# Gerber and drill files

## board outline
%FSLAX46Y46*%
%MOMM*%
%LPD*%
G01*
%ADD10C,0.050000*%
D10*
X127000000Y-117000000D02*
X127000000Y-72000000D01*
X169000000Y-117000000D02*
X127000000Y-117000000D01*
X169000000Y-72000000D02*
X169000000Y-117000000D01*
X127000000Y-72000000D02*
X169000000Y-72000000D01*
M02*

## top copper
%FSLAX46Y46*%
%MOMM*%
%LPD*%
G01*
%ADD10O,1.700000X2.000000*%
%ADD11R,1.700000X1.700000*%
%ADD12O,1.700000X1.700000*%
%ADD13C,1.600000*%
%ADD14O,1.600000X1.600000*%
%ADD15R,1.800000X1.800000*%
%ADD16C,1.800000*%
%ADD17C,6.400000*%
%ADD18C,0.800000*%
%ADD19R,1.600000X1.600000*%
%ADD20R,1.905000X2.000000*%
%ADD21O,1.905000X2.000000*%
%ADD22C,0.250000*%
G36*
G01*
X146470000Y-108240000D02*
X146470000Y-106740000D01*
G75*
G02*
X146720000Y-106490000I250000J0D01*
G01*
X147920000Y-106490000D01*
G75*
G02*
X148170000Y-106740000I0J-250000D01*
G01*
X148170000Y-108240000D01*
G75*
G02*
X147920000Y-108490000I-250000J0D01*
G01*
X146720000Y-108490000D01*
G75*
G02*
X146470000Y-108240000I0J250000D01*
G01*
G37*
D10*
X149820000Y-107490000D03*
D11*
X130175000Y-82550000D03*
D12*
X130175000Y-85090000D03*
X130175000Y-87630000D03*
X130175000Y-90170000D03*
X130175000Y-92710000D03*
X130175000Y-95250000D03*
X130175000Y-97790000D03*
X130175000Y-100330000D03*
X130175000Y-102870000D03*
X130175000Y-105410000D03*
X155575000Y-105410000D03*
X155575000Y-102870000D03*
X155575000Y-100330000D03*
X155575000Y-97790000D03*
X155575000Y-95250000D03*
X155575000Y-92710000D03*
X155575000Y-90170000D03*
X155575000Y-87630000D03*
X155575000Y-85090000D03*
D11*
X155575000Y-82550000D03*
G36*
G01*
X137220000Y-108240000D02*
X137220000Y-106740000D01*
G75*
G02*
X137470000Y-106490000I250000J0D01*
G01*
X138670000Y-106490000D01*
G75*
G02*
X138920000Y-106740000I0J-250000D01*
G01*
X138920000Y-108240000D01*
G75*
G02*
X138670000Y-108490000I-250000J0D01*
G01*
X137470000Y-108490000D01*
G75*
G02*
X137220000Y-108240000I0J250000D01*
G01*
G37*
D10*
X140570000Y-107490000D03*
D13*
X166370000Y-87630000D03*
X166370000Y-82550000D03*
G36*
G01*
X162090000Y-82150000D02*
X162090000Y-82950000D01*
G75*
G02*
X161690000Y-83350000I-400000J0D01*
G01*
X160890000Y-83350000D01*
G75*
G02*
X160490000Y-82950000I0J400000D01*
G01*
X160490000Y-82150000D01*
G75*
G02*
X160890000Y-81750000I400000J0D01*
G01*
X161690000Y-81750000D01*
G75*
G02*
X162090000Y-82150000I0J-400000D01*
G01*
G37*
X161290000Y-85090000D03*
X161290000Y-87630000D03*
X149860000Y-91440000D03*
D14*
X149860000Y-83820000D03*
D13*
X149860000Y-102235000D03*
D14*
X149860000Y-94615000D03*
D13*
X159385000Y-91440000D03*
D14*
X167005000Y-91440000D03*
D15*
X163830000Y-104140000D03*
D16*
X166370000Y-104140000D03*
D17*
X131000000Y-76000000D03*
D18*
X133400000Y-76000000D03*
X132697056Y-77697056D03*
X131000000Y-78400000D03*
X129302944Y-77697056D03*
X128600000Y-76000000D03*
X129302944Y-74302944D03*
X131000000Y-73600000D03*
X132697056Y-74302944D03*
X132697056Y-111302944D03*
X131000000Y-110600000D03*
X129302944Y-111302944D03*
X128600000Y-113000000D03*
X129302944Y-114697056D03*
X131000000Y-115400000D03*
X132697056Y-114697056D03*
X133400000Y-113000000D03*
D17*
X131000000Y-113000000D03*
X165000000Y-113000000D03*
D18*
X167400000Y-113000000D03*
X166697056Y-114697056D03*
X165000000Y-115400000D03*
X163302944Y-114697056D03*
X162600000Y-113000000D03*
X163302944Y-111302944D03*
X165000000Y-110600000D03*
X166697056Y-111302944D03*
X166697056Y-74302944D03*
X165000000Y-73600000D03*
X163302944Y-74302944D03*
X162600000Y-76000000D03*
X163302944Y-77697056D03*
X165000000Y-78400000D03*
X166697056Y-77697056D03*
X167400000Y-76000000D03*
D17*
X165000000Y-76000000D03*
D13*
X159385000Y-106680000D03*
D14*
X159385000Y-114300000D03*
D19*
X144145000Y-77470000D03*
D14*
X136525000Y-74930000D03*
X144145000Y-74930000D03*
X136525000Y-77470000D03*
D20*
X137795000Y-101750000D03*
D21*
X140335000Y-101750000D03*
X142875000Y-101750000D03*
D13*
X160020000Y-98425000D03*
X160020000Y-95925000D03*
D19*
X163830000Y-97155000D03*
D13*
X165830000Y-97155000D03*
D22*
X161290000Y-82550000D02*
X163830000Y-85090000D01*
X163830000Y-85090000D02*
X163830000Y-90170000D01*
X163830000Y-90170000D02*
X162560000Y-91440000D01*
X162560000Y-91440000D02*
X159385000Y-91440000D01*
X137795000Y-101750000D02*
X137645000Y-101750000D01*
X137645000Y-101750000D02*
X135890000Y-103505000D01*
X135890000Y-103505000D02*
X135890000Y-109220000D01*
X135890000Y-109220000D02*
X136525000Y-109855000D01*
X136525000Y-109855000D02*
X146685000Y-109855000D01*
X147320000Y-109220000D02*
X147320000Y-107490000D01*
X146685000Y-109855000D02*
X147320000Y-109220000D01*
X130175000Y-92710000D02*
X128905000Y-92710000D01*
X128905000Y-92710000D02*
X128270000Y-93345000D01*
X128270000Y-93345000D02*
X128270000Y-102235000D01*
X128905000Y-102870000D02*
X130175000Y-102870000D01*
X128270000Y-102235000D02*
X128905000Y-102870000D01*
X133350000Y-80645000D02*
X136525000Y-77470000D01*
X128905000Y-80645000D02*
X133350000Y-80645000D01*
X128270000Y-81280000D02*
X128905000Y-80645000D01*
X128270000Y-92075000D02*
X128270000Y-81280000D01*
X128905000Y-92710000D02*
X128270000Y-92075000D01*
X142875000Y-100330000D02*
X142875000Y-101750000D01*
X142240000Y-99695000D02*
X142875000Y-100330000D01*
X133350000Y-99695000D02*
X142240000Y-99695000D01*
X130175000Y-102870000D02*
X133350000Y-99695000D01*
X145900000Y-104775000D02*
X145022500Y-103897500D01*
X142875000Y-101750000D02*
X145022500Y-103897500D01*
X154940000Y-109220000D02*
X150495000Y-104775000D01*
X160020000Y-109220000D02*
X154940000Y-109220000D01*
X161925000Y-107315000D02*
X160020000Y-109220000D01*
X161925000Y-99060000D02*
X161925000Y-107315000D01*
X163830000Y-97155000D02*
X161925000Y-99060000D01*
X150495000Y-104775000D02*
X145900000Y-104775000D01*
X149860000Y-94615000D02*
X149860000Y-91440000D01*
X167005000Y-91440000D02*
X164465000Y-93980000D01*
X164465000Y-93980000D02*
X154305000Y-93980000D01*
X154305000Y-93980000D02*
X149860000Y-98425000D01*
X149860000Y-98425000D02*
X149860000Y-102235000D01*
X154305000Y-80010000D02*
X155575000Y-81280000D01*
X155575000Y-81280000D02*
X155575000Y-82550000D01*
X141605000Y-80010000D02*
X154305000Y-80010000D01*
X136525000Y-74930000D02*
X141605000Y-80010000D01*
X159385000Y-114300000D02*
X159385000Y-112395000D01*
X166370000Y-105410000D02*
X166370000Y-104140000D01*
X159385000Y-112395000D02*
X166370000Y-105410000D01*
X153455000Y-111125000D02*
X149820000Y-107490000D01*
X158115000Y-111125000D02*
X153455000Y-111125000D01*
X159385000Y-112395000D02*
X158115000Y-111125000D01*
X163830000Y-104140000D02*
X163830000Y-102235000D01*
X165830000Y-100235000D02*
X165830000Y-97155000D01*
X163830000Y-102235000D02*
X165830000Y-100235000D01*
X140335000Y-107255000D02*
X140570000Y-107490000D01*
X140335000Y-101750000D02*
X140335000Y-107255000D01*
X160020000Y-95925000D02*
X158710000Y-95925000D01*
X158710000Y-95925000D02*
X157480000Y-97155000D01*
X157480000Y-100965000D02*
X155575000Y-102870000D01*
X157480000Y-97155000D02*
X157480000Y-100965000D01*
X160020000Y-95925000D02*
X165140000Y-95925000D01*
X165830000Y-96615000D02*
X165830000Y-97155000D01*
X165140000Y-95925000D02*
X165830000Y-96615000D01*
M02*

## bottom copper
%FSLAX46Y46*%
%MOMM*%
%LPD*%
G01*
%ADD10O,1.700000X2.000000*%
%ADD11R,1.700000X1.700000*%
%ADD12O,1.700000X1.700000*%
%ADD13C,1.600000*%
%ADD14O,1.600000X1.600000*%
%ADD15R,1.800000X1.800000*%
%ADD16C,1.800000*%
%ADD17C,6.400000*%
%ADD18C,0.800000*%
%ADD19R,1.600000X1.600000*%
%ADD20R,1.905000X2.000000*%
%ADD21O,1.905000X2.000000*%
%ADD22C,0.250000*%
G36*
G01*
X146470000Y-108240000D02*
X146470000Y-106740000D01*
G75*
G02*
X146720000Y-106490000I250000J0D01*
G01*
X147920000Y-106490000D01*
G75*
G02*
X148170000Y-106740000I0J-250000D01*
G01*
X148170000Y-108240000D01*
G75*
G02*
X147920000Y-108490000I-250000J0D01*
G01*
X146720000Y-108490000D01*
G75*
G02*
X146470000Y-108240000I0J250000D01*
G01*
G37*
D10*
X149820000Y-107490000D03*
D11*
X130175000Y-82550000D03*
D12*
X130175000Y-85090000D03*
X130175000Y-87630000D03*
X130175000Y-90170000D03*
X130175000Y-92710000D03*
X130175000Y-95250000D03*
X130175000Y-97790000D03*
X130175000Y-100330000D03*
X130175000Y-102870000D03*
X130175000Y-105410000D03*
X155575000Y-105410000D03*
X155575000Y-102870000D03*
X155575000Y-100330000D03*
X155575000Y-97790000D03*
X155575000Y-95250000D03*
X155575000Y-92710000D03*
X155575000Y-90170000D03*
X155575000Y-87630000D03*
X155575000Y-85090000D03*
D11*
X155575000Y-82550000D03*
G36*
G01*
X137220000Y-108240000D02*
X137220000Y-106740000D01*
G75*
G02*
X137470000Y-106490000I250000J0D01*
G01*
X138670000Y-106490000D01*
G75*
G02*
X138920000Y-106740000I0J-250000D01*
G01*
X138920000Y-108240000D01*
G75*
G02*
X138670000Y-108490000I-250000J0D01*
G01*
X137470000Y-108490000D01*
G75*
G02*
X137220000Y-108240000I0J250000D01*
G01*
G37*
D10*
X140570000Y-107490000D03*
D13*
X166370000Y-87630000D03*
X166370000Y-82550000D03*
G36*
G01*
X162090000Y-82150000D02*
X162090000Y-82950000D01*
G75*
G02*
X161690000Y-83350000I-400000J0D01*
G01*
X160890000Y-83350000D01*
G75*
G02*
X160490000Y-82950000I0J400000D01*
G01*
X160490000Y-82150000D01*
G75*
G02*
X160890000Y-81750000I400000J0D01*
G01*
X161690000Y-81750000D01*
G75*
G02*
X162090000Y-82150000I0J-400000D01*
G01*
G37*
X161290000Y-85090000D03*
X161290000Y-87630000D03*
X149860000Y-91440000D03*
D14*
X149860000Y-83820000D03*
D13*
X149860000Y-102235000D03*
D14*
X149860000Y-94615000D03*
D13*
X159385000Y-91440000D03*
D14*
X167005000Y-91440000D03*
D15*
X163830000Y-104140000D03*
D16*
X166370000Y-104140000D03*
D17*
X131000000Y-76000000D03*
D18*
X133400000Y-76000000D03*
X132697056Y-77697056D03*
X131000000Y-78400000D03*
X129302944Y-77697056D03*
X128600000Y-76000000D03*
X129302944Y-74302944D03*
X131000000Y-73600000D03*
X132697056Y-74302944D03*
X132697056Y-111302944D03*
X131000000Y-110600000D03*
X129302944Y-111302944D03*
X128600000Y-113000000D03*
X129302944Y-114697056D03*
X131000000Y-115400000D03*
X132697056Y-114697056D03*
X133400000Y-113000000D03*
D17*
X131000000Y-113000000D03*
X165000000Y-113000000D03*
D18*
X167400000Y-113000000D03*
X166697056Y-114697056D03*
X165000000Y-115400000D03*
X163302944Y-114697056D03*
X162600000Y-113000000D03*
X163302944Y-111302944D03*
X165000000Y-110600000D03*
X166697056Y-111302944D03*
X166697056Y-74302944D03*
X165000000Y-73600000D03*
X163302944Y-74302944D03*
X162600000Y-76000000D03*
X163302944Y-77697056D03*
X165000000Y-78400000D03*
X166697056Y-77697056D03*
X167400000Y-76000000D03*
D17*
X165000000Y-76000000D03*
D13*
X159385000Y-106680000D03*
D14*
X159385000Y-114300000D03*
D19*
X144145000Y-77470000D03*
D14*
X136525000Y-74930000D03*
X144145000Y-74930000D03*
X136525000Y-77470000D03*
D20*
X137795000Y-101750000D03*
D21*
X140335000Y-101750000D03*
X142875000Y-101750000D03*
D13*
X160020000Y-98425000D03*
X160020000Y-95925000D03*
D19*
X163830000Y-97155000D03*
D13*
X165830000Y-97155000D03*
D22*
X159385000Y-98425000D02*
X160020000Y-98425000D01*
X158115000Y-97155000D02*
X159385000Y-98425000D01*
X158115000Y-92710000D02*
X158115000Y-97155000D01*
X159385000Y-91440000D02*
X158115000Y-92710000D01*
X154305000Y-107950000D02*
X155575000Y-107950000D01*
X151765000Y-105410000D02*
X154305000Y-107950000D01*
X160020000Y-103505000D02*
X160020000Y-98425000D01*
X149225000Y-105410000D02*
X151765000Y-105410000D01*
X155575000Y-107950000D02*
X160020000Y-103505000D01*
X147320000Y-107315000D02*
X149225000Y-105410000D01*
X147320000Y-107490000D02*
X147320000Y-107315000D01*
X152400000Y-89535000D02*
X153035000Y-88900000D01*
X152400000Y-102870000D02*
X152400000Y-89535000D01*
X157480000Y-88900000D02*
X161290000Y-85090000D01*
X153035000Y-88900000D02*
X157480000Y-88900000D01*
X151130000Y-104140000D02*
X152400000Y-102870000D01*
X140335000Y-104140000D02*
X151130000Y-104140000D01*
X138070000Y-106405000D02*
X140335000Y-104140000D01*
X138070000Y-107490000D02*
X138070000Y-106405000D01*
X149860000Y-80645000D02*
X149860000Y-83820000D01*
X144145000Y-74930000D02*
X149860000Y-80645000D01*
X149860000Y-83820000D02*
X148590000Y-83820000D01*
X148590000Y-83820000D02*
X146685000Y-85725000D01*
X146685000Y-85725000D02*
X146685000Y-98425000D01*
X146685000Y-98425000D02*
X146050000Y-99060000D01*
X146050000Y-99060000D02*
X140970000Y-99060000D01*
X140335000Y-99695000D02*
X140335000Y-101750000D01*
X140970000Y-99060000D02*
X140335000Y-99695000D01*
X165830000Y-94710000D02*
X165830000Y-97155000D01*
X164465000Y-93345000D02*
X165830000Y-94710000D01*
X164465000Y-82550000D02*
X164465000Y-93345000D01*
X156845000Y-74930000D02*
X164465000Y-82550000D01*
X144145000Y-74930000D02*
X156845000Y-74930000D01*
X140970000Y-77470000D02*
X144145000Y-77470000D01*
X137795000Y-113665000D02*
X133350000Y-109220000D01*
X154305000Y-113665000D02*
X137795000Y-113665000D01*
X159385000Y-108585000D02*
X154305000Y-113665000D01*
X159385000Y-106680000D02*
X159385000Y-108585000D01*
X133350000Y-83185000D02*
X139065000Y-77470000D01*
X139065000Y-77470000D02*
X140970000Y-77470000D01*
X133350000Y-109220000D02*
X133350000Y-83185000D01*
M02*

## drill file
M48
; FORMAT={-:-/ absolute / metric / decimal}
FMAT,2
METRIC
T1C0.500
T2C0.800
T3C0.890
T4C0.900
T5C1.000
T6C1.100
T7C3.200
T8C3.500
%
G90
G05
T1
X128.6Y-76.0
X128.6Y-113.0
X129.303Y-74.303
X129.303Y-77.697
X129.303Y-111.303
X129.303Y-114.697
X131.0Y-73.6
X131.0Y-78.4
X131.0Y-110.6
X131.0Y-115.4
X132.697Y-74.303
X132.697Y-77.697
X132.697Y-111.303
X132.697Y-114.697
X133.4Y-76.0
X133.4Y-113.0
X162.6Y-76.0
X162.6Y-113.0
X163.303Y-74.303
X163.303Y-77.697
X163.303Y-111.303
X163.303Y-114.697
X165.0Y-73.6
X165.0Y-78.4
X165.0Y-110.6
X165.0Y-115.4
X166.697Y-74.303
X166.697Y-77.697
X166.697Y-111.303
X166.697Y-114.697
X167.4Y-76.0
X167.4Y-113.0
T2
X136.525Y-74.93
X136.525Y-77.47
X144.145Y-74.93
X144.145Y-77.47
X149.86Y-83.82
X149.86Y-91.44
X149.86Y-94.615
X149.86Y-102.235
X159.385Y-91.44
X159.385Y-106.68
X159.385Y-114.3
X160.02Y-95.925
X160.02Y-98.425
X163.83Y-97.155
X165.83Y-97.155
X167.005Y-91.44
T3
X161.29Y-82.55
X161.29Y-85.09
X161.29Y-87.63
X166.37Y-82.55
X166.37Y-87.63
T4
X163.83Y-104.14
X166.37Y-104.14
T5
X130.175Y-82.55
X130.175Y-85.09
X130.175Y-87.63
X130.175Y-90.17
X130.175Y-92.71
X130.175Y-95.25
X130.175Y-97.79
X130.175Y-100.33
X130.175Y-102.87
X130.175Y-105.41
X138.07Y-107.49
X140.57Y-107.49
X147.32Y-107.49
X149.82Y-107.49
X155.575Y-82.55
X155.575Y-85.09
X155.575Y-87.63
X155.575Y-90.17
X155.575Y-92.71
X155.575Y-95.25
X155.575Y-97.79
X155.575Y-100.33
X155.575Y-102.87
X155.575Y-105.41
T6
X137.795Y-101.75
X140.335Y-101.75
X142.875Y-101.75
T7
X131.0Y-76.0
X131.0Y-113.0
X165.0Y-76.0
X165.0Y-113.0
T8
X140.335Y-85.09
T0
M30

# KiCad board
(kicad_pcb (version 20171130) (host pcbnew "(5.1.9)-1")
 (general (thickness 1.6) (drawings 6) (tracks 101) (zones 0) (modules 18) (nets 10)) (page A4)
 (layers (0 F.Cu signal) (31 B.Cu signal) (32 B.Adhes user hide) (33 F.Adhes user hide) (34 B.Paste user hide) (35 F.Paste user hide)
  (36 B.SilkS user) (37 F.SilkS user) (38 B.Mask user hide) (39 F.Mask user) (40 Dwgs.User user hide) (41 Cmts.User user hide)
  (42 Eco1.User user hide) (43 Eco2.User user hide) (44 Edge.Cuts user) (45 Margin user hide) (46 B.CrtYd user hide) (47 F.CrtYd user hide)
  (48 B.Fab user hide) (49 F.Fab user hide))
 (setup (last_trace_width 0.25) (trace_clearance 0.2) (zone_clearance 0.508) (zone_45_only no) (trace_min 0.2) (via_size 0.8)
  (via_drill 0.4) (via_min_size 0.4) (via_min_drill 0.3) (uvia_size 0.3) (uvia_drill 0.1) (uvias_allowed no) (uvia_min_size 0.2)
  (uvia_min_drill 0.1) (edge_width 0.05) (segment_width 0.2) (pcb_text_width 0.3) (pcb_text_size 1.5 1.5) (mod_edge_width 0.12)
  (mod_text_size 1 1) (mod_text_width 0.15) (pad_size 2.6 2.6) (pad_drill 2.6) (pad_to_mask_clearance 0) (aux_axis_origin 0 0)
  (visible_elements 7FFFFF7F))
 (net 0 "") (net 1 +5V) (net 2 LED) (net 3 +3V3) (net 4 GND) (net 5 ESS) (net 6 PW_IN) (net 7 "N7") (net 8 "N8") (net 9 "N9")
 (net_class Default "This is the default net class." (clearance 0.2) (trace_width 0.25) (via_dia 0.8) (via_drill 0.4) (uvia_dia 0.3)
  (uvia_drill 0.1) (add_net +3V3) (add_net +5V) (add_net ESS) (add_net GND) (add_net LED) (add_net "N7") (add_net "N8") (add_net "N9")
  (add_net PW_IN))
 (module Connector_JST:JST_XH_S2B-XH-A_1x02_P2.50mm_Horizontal (layer F.Cu) (at 147.32 107.49)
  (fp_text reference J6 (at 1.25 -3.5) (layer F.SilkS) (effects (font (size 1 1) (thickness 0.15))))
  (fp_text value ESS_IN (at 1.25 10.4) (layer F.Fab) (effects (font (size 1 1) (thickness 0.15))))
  (pad 1 thru_hole roundrect (at 0 0) (size 1.7 2) (drill 1) (layers *.Cu *.Mask) (roundrect_rratio 0.1470588235294118) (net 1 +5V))
  (pad 2 thru_hole oval (at 2.5 0) (size 1.7 2) (drill 1) (layers *.Cu *.Mask) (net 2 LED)))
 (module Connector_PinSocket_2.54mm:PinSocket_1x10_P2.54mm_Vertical (layer F.Cu) (at 130.175 82.55)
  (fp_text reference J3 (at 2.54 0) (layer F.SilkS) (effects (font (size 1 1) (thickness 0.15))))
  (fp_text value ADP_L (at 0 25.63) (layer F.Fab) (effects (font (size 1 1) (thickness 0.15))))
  (pad 1 thru_hole rect (at 0 0) (size 1.7 1.7) (drill 1) (layers *.Cu *.Mask))
  (pad 2 thru_hole oval (at 0 2.54) (size 1.7 1.7) (drill 1) (layers *.Cu *.Mask))
  (pad 3 thru_hole oval (at 0 5.08) (size 1.7 1.7) (drill 1) (layers *.Cu *.Mask))
  (pad 4 thru_hole oval (at 0 7.62) (size 1.7 1.7) (drill 1) (layers *.Cu *.Mask))
  (pad 5 thru_hole oval (at 0 10.16) (size 1.7 1.7) (drill 1) (layers *.Cu *.Mask) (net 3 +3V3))
  (pad 6 thru_hole oval (at 0 12.7) (size 1.7 1.7) (drill 1) (layers *.Cu *.Mask))
  (pad 7 thru_hole oval (at 0 15.24) (size 1.7 1.7) (drill 1) (layers *.Cu *.Mask))
  (pad 8 thru_hole oval (at 0 17.78) (size 1.7 1.7) (drill 1) (layers *.Cu *.Mask))
  (pad 9 thru_hole oval (at 0 20.32) (size 1.7 1.7) (drill 1) (layers *.Cu *.Mask) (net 3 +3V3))
  (pad 10 thru_hole oval (at 0 22.86) (size 1.7 1.7) (drill 1) (layers *.Cu *.Mask)))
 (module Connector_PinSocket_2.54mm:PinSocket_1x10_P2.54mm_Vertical (layer F.Cu) (at 155.575 82.55)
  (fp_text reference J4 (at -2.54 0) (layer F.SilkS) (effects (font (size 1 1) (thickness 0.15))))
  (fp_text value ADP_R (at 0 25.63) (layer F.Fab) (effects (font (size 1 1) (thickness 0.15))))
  (pad 10 thru_hole oval (at 0 22.86) (size 1.7 1.7) (drill 1) (layers *.Cu *.Mask))
  (pad 9 thru_hole oval (at 0 20.32) (size 1.7 1.7) (drill 1) (layers *.Cu *.Mask) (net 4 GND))
  (pad 8 thru_hole oval (at 0 17.78) (size 1.7 1.7) (drill 1) (layers *.Cu *.Mask))
  (pad 7 thru_hole oval (at 0 15.24) (size 1.7 1.7) (drill 1) (layers *.Cu *.Mask))
  (pad 6 thru_hole oval (at 0 12.7) (size 1.7 1.7) (drill 1) (layers *.Cu *.Mask))
  (pad 5 thru_hole oval (at 0 10.16) (size 1.7 1.7) (drill 1) (layers *.Cu *.Mask))
  (pad 4 thru_hole oval (at 0 7.62) (size 1.7 1.7) (drill 1) (layers *.Cu *.Mask))
  (pad 3 thru_hole oval (at 0 5.08) (size 1.7 1.7) (drill 1) (layers *.Cu *.Mask))
  (pad 2 thru_hole oval (at 0 2.54) (size 1.7 1.7) (drill 1) (layers *.Cu *.Mask))
  (pad 1 thru_hole rect (at 0 0) (size 1.7 1.7) (drill 1) (layers *.Cu *.Mask) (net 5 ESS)))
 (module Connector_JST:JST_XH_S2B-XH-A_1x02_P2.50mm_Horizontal (layer F.Cu) (at 138.07 107.49)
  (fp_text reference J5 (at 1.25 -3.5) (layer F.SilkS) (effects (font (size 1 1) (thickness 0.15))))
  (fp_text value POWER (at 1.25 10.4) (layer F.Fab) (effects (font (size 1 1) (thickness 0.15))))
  (pad 1 thru_hole roundrect (at 0 0) (size 1.7 2) (drill 1) (layers *.Cu *.Mask) (roundrect_rratio 0.1470588235294118) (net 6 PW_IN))
  (pad 2 thru_hole oval (at 2.5 0) (size 1.7 2) (drill 1) (layers *.Cu *.Mask) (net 4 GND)))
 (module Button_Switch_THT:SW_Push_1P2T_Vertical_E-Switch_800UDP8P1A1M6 (layer F.Cu) (at 161.29 82.55)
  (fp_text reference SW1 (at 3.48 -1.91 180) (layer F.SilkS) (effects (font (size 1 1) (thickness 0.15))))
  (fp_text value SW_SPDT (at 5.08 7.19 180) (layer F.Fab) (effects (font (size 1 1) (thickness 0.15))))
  (pad "" thru_hole circle (at 5.08 5.08 180) (size 1.6 1.6) (drill 0.89) (layers *.Cu *.Mask))
  (pad "" thru_hole circle (at 5.08 0 180) (size 1.6 1.6) (drill 0.89) (layers *.Cu *.Mask))
  (pad 1 thru_hole roundrect (at 0 0 180) (size 1.6 1.6) (drill 0.89) (layers *.Cu *.Mask) (roundrect_rratio 0.25) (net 1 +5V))
  (pad 2 thru_hole circle (at 0 2.54 180) (size 1.6 1.6) (drill 0.89) (layers *.Cu *.Mask) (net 6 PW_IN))
  (pad 3 thru_hole circle (at 0 5.08 180) (size 1.6 1.6) (drill 0.89) (layers *.Cu *.Mask)))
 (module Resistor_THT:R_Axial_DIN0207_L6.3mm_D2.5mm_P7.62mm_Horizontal (layer F.Cu) (at 149.86 91.44 90)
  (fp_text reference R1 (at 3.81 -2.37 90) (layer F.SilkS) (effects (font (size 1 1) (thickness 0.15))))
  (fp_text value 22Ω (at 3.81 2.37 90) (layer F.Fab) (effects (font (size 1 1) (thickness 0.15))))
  (pad 1 thru_hole circle (at 0 0 90) (size 1.6 1.6) (drill 0.8) (layers *.Cu *.Mask) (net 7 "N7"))
  (pad 2 thru_hole oval (at 7.62 0 90) (size 1.6 1.6) (drill 0.8) (layers *.Cu *.Mask) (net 4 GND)))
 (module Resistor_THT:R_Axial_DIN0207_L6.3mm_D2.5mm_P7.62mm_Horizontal (layer F.Cu) (at 149.86 102.235 90)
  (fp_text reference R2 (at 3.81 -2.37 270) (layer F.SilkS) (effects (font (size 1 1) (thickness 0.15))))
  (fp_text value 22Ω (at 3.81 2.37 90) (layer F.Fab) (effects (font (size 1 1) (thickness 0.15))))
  (pad 1 thru_hole circle (at 0 0 90) (size 1.6 1.6) (drill 0.8) (layers *.Cu *.Mask) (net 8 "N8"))
  (pad 2 thru_hole oval (at 7.62 0 90) (size 1.6 1.6) (drill 0.8) (layers *.Cu *.Mask) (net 7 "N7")))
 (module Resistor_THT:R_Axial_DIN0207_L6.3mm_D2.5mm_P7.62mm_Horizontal (layer F.Cu) (at 159.385 91.44)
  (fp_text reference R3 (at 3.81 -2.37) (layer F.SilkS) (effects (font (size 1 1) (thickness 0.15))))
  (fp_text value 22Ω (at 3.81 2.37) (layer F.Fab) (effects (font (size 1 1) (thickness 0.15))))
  (pad 1 thru_hole circle (at 0 0) (size 1.6 1.6) (drill 0.8) (layers *.Cu *.Mask) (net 1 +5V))
  (pad 2 thru_hole oval (at 7.62 0) (size 1.6 1.6) (drill 0.8) (layers *.Cu *.Mask) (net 8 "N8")))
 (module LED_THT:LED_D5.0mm (layer F.Cu) (at 163.83 104.14)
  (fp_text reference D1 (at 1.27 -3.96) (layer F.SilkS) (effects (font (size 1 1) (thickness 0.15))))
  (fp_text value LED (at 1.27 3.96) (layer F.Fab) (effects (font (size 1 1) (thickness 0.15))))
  (pad 1 thru_hole rect (at 0 0) (size 1.8 1.8) (drill 0.9) (layers *.Cu *.Mask) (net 4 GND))
  (pad 2 thru_hole circle (at 2.54 0) (size 1.8 1.8) (drill 0.9) (layers *.Cu *.Mask) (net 2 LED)))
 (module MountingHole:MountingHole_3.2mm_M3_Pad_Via (layer F.Cu) (at 131 76)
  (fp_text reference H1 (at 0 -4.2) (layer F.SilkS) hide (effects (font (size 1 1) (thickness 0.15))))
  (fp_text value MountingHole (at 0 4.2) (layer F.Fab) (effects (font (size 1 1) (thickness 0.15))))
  (pad 1 thru_hole circle (at 0 0) (size 6.4 6.4) (drill 3.2) (layers *.Cu *.Mask))
  (pad 1 thru_hole circle (at 2.4 0) (size 0.8 0.8) (drill 0.5) (layers *.Cu *.Mask))
  (pad 1 thru_hole circle (at 1.697056 1.697056) (size 0.8 0.8) (drill 0.5) (layers *.Cu *.Mask))
  (pad 1 thru_hole circle (at 0 2.4) (size 0.8 0.8) (drill 0.5) (layers *.Cu *.Mask))
  (pad 1 thru_hole circle (at -1.697056 1.697056) (size 0.8 0.8) (drill 0.5) (layers *.Cu *.Mask))
  (pad 1 thru_hole circle (at -2.4 0) (size 0.8 0.8) (drill 0.5) (layers *.Cu *.Mask))
  (pad 1 thru_hole circle (at -1.697056 -1.697056) (size 0.8 0.8) (drill 0.5) (layers *.Cu *.Mask))
  (pad 1 thru_hole circle (at 0 -2.4) (size 0.8 0.8) (drill 0.5) (layers *.Cu *.Mask))
  (pad 1 thru_hole circle (at 1.697056 -1.697056) (size 0.8 0.8) (drill 0.5) (layers *.Cu *.Mask)))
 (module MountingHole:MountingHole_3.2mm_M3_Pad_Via (layer F.Cu) (at 131 113)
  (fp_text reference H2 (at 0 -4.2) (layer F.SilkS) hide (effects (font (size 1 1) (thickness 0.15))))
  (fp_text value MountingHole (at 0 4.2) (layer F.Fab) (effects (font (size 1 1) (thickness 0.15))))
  (pad 1 thru_hole circle (at 1.697056 -1.697056) (size 0.8 0.8) (drill 0.5) (layers *.Cu *.Mask))
  (pad 1 thru_hole circle (at 0 -2.4) (size 0.8 0.8) (drill 0.5) (layers *.Cu *.Mask))
  (pad 1 thru_hole circle (at -1.697056 -1.697056) (size 0.8 0.8) (drill 0.5) (layers *.Cu *.Mask))
  (pad 1 thru_hole circle (at -2.4 0) (size 0.8 0.8) (drill 0.5) (layers *.Cu *.Mask))
  (pad 1 thru_hole circle (at -1.697056 1.697056) (size 0.8 0.8) (drill 0.5) (layers *.Cu *.Mask))
  (pad 1 thru_hole circle (at 0 2.4) (size 0.8 0.8) (drill 0.5) (layers *.Cu *.Mask))
  (pad 1 thru_hole circle (at 1.697056 1.697056) (size 0.8 0.8) (drill 0.5) (layers *.Cu *.Mask))
  (pad 1 thru_hole circle (at 2.4 0) (size 0.8 0.8) (drill 0.5) (layers *.Cu *.Mask))
  (pad 1 thru_hole circle (at 0 0) (size 6.4 6.4) (drill 3.2) (layers *.Cu *.Mask)))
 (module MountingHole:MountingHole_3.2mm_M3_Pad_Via (layer F.Cu) (at 165 113)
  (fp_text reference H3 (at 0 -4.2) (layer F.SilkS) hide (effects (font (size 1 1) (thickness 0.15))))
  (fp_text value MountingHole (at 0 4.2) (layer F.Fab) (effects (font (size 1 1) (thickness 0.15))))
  (pad 1 thru_hole circle (at 0 0) (size 6.4 6.4) (drill 3.2) (layers *.Cu *.Mask))
  (pad 1 thru_hole circle (at 2.4 0) (size 0.8 0.8) (drill 0.5) (layers *.Cu *.Mask))
  (pad 1 thru_hole circle (at 1.697056 1.697056) (size 0.8 0.8) (drill 0.5) (layers *.Cu *.Mask))
  (pad 1 thru_hole circle (at 0 2.4) (size 0.8 0.8) (drill 0.5) (layers *.Cu *.Mask))
  (pad 1 thru_hole circle (at -1.697056 1.697056) (size 0.8 0.8) (drill 0.5) (layers *.Cu *.Mask))
  (pad 1 thru_hole circle (at -2.4 0) (size 0.8 0.8) (drill 0.5) (layers *.Cu *.Mask))
  (pad 1 thru_hole circle (at -1.697056 -1.697056) (size 0.8 0.8) (drill 0.5) (layers *.Cu *.Mask))
  (pad 1 thru_hole circle (at 0 -2.4) (size 0.8 0.8) (drill 0.5) (layers *.Cu *.Mask))
  (pad 1 thru_hole circle (at 1.697056 -1.697056) (size 0.8 0.8) (drill 0.5) (layers *.Cu *.Mask)))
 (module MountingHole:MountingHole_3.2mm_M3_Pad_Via (layer F.Cu) (at 165 76)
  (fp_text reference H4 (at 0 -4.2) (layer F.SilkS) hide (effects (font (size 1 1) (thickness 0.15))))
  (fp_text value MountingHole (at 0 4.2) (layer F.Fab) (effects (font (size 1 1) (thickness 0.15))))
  (pad 1 thru_hole circle (at 1.697056 -1.697056) (size 0.8 0.8) (drill 0.5) (layers *.Cu *.Mask))
  (pad 1 thru_hole circle (at 0 -2.4) (size 0.8 0.8) (drill 0.5) (layers *.Cu *.Mask))
  (pad 1 thru_hole circle (at -1.697056 -1.697056) (size 0.8 0.8) (drill 0.5) (layers *.Cu *.Mask))
  (pad 1 thru_hole circle (at -2.4 0) (size 0.8 0.8) (drill 0.5) (layers *.Cu *.Mask))
  (pad 1 thru_hole circle (at -1.697056 1.697056) (size 0.8 0.8) (drill 0.5) (layers *.Cu *.Mask))
  (pad 1 thru_hole circle (at 0 2.4) (size 0.8 0.8) (drill 0.5) (layers *.Cu *.Mask))
  (pad 1 thru_hole circle (at 1.697056 1.697056) (size 0.8 0.8) (drill 0.5) (layers *.Cu *.Mask))
  (pad 1 thru_hole circle (at 2.4 0) (size 0.8 0.8) (drill 0.5) (layers *.Cu *.Mask))
  (pad 1 thru_hole circle (at 0 0) (size 6.4 6.4) (drill 3.2) (layers *.Cu *.Mask)))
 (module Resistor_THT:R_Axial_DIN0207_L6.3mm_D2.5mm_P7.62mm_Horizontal (layer F.Cu) (at 159.385 106.68 270)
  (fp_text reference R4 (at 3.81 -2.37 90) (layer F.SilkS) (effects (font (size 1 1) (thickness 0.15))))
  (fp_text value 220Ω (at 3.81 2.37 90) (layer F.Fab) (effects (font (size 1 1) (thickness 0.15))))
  (pad 1 thru_hole circle (at 0 0 270) (size 1.6 1.6) (drill 0.8) (layers *.Cu *.Mask) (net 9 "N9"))
  (pad 2 thru_hole oval (at 7.62 0 270) (size 1.6 1.6) (drill 0.8) (layers *.Cu *.Mask) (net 2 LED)))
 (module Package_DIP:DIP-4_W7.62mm (layer F.Cu) (at 144.145 77.47 180)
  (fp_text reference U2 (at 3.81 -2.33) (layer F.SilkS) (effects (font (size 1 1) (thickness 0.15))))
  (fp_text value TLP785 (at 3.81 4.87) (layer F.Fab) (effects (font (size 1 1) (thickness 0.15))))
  (pad 1 thru_hole rect (at 0 0 180) (size 1.6 1.6) (drill 0.8) (layers *.Cu *.Mask) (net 9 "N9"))
  (pad 3 thru_hole oval (at 7.62 2.54 180) (size 1.6 1.6) (drill 0.8) (layers *.Cu *.Mask) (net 5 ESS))
  (pad 2 thru_hole oval (at 0 2.54 180) (size 1.6 1.6) (drill 0.8) (layers *.Cu *.Mask) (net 4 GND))
  (pad 4 thru_hole oval (at 7.62 0 180) (size 1.6 1.6) (drill 0.8) (layers *.Cu *.Mask) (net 3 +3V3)))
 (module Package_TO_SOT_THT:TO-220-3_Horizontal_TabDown (layer F.Cu) (at 137.795 101.75)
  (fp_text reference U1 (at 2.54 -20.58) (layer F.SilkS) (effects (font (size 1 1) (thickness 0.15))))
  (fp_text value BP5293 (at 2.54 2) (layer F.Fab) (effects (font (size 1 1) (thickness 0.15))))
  (pad "" np_thru_hole oval (at 2.54 -16.66) (size 3.5 3.5) (drill 3.5) (layers *.Cu *.Mask))
  (pad 1 thru_hole rect (at 0 0) (size 1.905 2) (drill 1.1) (layers *.Cu *.Mask) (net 1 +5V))
  (pad 2 thru_hole oval (at 2.54 0) (size 1.905 2) (drill 1.1) (layers *.Cu *.Mask) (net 4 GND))
  (pad 3 thru_hole oval (at 5.08 0) (size 1.905 2) (drill 1.1) (layers *.Cu *.Mask) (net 3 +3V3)))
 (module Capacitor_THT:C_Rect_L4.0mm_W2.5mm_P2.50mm (layer F.Cu) (at 160.02 98.425 90)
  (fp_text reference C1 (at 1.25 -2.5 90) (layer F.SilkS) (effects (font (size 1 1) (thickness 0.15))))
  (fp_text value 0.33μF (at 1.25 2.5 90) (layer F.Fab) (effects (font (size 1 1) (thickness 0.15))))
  (pad 1 thru_hole circle (at 0 0 90) (size 1.6 1.6) (drill 0.8) (layers *.Cu *.Mask) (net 1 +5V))
  (pad 2 thru_hole circle (at 2.5 0 90) (size 1.6 1.6) (drill 0.8) (layers *.Cu *.Mask) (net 4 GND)))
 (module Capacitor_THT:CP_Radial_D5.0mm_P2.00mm (layer F.Cu) (at 163.83 97.155)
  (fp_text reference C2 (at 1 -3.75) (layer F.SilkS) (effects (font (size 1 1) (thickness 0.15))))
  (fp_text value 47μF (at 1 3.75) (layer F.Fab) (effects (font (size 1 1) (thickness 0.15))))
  (pad 1 thru_hole rect (at 0 0) (size 1.6 1.6) (drill 0.8) (layers *.Cu *.Mask) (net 3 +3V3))
  (pad 2 thru_hole circle (at 2 0) (size 1.6 1.6) (drill 0.8) (layers *.Cu *.Mask) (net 4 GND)))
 (gr_line (start 127 117) (end 127 72) (layer Edge.Cuts) (width 0.05))
 (gr_line (start 169 117) (end 127 117) (layer Edge.Cuts) (width 0.05))
 (gr_line (start 169 72) (end 169 117) (layer Edge.Cuts) (width 0.05))
 (gr_line (start 127 72) (end 169 72) (layer Edge.Cuts) (width 0.05))
 (segment (start 161.29 82.55) (end 163.83 85.09) (width 0.25) (layer F.Cu) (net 1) (status 10))
 (segment (start 163.83 85.09) (end 163.83 90.17) (width 0.25) (layer F.Cu) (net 1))
 (segment (start 163.83 90.17) (end 162.56 91.44) (width 0.25) (layer F.Cu) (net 1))
 (segment (start 162.56 91.44) (end 159.385 91.44) (width 0.25) (layer F.Cu) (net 1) (status 20))
 (segment (start 137.795 101.75) (end 137.645 101.75) (width 0.25) (layer F.Cu) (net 1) (status 30))
 (segment (start 137.645 101.75) (end 135.89 103.505) (width 0.25) (layer F.Cu) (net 1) (status 10))
 (segment (start 135.89 103.505) (end 135.89 109.22) (width 0.25) (layer F.Cu) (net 1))
 (segment (start 135.89 109.22) (end 136.525 109.855) (width 0.25) (layer F.Cu) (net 1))
 (segment (start 136.525 109.855) (end 146.685 109.855) (width 0.25) (layer F.Cu) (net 1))
 (segment (start 147.32 109.22) (end 147.32 107.49) (width 0.25) (layer F.Cu) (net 1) (status 20))
 (segment (start 146.685 109.855) (end 147.32 109.22) (width 0.25) (layer F.Cu) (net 1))
 (segment (start 159.385 98.425) (end 160.02 98.425) (width 0.25) (layer B.Cu) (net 1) (status 30))
 (segment (start 158.115 97.155) (end 159.385 98.425) (width 0.25) (layer B.Cu) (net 1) (status 20))
 (segment (start 158.115 92.71) (end 158.115 97.155) (width 0.25) (layer B.Cu) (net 1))
 (segment (start 159.385 91.44) (end 158.115 92.71) (width 0.25) (layer B.Cu) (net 1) (status 10))
 (segment (start 154.305 107.95) (end 155.575 107.95) (width 0.25) (layer B.Cu) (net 1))
 (segment (start 151.765 105.41) (end 154.305 107.95) (width 0.25) (layer B.Cu) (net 1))
 (segment (start 160.02 103.505) (end 160.02 98.425) (width 0.25) (layer B.Cu) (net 1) (status 20))
 (segment (start 149.225 105.41) (end 151.765 105.41) (width 0.25) (layer B.Cu) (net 1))
 (segment (start 155.575 107.95) (end 160.02 103.505) (width 0.25) (layer B.Cu) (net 1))
 (segment (start 147.32 107.315) (end 149.225 105.41) (width 0.25) (layer B.Cu) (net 1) (status 10))
 (segment (start 147.32 107.49) (end 147.32 107.315) (width 0.25) (layer B.Cu) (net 1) (status 30))
 (segment (start 130.175 92.71) (end 128.905 92.71) (width 0.25) (layer F.Cu) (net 3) (status 10))
 (segment (start 128.905 92.71) (end 128.27 93.345) (width 0.25) (layer F.Cu) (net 3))
 (segment (start 128.27 93.345) (end 128.27 102.235) (width 0.25) (layer F.Cu) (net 3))
 (segment (start 128.905 102.87) (end 130.175 102.87) (width 0.25) (layer F.Cu) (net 3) (status 20))
 (segment (start 128.27 102.235) (end 128.905 102.87) (width 0.25) (layer F.Cu) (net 3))
 (segment (start 133.35 80.645) (end 136.525 77.47) (width 0.25) (layer F.Cu) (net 3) (status 20))
 (segment (start 128.905 80.645) (end 133.35 80.645) (width 0.25) (layer F.Cu) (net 3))
 (segment (start 128.27 81.28) (end 128.905 80.645) (width 0.25) (layer F.Cu) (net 3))
 (segment (start 128.27 92.075) (end 128.27 81.28) (width 0.25) (layer F.Cu) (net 3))
 (segment (start 128.905 92.71) (end 128.27 92.075) (width 0.25) (layer F.Cu) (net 3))
 (segment (start 142.875 100.33) (end 142.875 101.75) (width 0.25) (layer F.Cu) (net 3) (status 20))
 (segment (start 142.24 99.695) (end 142.875 100.33) (width 0.25) (layer F.Cu) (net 3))
 (segment (start 133.35 99.695) (end 142.24 99.695) (width 0.25) (layer F.Cu) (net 3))
 (segment (start 130.175 102.87) (end 133.35 99.695) (width 0.25) (layer F.Cu) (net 3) (status 10))
 (segment (start 145.9 104.775) (end 145.0225 103.8975) (width 0.25) (layer F.Cu) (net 3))
 (segment (start 142.875 101.75) (end 145.0225 103.8975) (width 0.25) (layer F.Cu) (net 3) (status 10))
 (segment (start 154.94 109.22) (end 150.495 104.775) (width 0.25) (layer F.Cu) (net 3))
 (segment (start 160.02 109.22) (end 154.94 109.22) (width 0.25) (layer F.Cu) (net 3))
 (segment (start 161.925 107.315) (end 160.02 109.22) (width 0.25) (layer F.Cu) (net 3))
 (segment (start 161.925 99.06) (end 161.925 107.315) (width 0.25) (layer F.Cu) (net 3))
 (segment (start 163.83 97.155) (end 161.925 99.06) (width 0.25) (layer F.Cu) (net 3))
 (segment (start 150.495 104.775) (end 145.9 104.775) (width 0.25) (layer F.Cu) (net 3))
 (segment (start 152.4 89.535) (end 153.035 88.9) (width 0.25) (layer B.Cu) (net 6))
 (segment (start 152.4 102.87) (end 152.4 89.535) (width 0.25) (layer B.Cu) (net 6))
 (segment (start 157.48 88.9) (end 161.29 85.09) (width 0.25) (layer B.Cu) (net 6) (status 20))
 (segment (start 153.035 88.9) (end 157.48 88.9) (width 0.25) (layer B.Cu) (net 6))
 (segment (start 151.13 104.14) (end 152.4 102.87) (width 0.25) (layer B.Cu) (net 6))
 (segment (start 140.335 104.14) (end 151.13 104.14) (width 0.25) (layer B.Cu) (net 6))
 (segment (start 138.07 106.405) (end 140.335 104.14) (width 0.25) (layer B.Cu) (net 6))
 (segment (start 138.07 107.49) (end 138.07 106.405) (width 0.25) (layer B.Cu) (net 6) (status 10))
 (segment (start 149.86 94.615) (end 149.86 91.44) (width 0.25) (layer F.Cu) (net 7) (status 30))
 (segment (start 167.005 91.44) (end 164.465 93.98) (width 0.25) (layer F.Cu) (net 8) (status 10))
 (segment (start 164.465 93.98) (end 154.305 93.98) (width 0.25) (layer F.Cu) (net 8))
 (segment (start 154.305 93.98) (end 149.86 98.425) (width 0.25) (layer F.Cu) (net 8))
 (segment (start 149.86 98.425) (end 149.86 102.235) (width 0.25) (layer F.Cu) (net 8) (status 20))
 (segment (start 154.305 80.01) (end 155.575 81.28) (width 0.25) (layer F.Cu) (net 5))
 (segment (start 155.575 81.28) (end 155.575 82.55) (width 0.25) (layer F.Cu) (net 5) (status 20))
 (segment (start 141.605 80.01) (end 154.305 80.01) (width 0.25) (layer F.Cu) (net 5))
 (segment (start 136.525 74.93) (end 141.605 80.01) (width 0.25) (layer F.Cu) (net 5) (status 10))
 (segment (start 159.385 114.3) (end 159.385 112.395) (width 0.25) (layer F.Cu) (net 2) (status 10))
 (segment (start 166.37 105.41) (end 166.37 104.14) (width 0.25) (layer F.Cu) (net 2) (status 20))
 (segment (start 159.385 112.395) (end 166.37 105.41) (width 0.25) (layer F.Cu) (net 2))
 (segment (start 153.455 111.125) (end 149.82 107.49) (width 0.25) (layer F.Cu) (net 2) (status 20))
 (segment (start 158.115 111.125) (end 153.455 111.125) (width 0.25) (layer F.Cu) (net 2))
 (segment (start 159.385 112.395) (end 158.115 111.125) (width 0.25) (layer F.Cu) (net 2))
 (segment (start 163.83 104.14) (end 163.83 102.235) (width 0.25) (layer F.Cu) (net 4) (status 10))
 (segment (start 165.83 100.235) (end 165.83 97.155) (width 0.25) (layer F.Cu) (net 4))
 (segment (start 163.83 102.235) (end 165.83 100.235) (width 0.25) (layer F.Cu) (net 4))
 (segment (start 140.335 107.255) (end 140.57 107.49) (width 0.25) (layer F.Cu) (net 4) (status 30))
 (segment (start 140.335 101.75) (end 140.335 107.255) (width 0.25) (layer F.Cu) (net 4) (status 30))
 (segment (start 149.86 80.645) (end 149.86 83.82) (width 0.25) (layer B.Cu) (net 4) (status 20))
 (segment (start 144.145 74.93) (end 149.86 80.645) (width 0.25) (layer B.Cu) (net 4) (status 10))
 (segment (start 160.02 95.925) (end 158.71 95.925) (width 0.25) (layer F.Cu) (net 4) (status 10))
 (segment (start 158.71 95.925) (end 157.48 97.155) (width 0.25) (layer F.Cu) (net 4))
 (segment (start 157.48 100.965) (end 155.575 102.87) (width 0.25) (layer F.Cu) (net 4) (status 20))
 (segment (start 157.48 97.155) (end 157.48 100.965) (width 0.25) (layer F.Cu) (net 4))
 (segment (start 149.86 83.82) (end 148.59 83.82) (width 0.25) (layer B.Cu) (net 4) (status 10))
 (segment (start 148.59 83.82) (end 146.685 85.725) (width 0.25) (layer B.Cu) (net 4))
 (segment (start 146.685 85.725) (end 146.685 98.425) (width 0.25) (layer B.Cu) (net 4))
 (segment (start 146.685 98.425) (end 146.05 99.06) (width 0.25) (layer B.Cu) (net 4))
 (segment (start 146.05 99.06) (end 140.97 99.06) (width 0.25) (layer B.Cu) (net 4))
 (segment (start 140.335 99.695) (end 140.335 101.75) (width 0.25) (layer B.Cu) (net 4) (status 20))
 (segment (start 140.97 99.06) (end 140.335 99.695) (width 0.25) (layer B.Cu) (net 4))
 (segment (start 165.83 94.71) (end 165.83 97.155) (width 0.25) (layer B.Cu) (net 4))
 (segment (start 164.465 93.345) (end 165.83 94.71) (width 0.25) (layer B.Cu) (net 4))
 (segment (start 164.465 82.55) (end 164.465 93.345) (width 0.25) (layer B.Cu) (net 4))
 (segment (start 156.845 74.93) (end 164.465 82.55) (width 0.25) (layer B.Cu) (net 4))
 (segment (start 144.145 74.93) (end 156.845 74.93) (width 0.25) (layer B.Cu) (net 4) (status 10))
 (segment (start 160.02 95.925) (end 165.14 95.925) (width 0.25) (layer F.Cu) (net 4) (status 10))
 (segment (start 165.83 96.615) (end 165.83 97.155) (width 0.25) (layer F.Cu) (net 4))
 (segment (start 165.14 95.925) (end 165.83 96.615) (width 0.25) (layer F.Cu) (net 4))
 (segment (start 140.97 77.47) (end 144.145 77.47) (width 0.25) (layer B.Cu) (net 9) (status 20))
 (segment (start 137.795 113.665) (end 133.35 109.22) (width 0.25) (layer B.Cu) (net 9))
 (segment (start 154.305 113.665) (end 137.795 113.665) (width 0.25) (layer B.Cu) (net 9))
 (segment (start 159.385 108.585) (end 154.305 113.665) (width 0.25) (layer B.Cu) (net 9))
 (segment (start 159.385 106.68) (end 159.385 108.585) (width 0.25) (layer B.Cu) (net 9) (status 10))
 (segment (start 133.35 83.185) (end 139.065 77.47) (width 0.25) (layer B.Cu) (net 9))
 (segment (start 139.065 77.47) (end 140.97 77.47) (width 0.25) (layer B.Cu) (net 9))
 (segment (start 133.35 109.22) (end 133.35 83.185) (width 0.25) (layer B.Cu) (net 9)))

